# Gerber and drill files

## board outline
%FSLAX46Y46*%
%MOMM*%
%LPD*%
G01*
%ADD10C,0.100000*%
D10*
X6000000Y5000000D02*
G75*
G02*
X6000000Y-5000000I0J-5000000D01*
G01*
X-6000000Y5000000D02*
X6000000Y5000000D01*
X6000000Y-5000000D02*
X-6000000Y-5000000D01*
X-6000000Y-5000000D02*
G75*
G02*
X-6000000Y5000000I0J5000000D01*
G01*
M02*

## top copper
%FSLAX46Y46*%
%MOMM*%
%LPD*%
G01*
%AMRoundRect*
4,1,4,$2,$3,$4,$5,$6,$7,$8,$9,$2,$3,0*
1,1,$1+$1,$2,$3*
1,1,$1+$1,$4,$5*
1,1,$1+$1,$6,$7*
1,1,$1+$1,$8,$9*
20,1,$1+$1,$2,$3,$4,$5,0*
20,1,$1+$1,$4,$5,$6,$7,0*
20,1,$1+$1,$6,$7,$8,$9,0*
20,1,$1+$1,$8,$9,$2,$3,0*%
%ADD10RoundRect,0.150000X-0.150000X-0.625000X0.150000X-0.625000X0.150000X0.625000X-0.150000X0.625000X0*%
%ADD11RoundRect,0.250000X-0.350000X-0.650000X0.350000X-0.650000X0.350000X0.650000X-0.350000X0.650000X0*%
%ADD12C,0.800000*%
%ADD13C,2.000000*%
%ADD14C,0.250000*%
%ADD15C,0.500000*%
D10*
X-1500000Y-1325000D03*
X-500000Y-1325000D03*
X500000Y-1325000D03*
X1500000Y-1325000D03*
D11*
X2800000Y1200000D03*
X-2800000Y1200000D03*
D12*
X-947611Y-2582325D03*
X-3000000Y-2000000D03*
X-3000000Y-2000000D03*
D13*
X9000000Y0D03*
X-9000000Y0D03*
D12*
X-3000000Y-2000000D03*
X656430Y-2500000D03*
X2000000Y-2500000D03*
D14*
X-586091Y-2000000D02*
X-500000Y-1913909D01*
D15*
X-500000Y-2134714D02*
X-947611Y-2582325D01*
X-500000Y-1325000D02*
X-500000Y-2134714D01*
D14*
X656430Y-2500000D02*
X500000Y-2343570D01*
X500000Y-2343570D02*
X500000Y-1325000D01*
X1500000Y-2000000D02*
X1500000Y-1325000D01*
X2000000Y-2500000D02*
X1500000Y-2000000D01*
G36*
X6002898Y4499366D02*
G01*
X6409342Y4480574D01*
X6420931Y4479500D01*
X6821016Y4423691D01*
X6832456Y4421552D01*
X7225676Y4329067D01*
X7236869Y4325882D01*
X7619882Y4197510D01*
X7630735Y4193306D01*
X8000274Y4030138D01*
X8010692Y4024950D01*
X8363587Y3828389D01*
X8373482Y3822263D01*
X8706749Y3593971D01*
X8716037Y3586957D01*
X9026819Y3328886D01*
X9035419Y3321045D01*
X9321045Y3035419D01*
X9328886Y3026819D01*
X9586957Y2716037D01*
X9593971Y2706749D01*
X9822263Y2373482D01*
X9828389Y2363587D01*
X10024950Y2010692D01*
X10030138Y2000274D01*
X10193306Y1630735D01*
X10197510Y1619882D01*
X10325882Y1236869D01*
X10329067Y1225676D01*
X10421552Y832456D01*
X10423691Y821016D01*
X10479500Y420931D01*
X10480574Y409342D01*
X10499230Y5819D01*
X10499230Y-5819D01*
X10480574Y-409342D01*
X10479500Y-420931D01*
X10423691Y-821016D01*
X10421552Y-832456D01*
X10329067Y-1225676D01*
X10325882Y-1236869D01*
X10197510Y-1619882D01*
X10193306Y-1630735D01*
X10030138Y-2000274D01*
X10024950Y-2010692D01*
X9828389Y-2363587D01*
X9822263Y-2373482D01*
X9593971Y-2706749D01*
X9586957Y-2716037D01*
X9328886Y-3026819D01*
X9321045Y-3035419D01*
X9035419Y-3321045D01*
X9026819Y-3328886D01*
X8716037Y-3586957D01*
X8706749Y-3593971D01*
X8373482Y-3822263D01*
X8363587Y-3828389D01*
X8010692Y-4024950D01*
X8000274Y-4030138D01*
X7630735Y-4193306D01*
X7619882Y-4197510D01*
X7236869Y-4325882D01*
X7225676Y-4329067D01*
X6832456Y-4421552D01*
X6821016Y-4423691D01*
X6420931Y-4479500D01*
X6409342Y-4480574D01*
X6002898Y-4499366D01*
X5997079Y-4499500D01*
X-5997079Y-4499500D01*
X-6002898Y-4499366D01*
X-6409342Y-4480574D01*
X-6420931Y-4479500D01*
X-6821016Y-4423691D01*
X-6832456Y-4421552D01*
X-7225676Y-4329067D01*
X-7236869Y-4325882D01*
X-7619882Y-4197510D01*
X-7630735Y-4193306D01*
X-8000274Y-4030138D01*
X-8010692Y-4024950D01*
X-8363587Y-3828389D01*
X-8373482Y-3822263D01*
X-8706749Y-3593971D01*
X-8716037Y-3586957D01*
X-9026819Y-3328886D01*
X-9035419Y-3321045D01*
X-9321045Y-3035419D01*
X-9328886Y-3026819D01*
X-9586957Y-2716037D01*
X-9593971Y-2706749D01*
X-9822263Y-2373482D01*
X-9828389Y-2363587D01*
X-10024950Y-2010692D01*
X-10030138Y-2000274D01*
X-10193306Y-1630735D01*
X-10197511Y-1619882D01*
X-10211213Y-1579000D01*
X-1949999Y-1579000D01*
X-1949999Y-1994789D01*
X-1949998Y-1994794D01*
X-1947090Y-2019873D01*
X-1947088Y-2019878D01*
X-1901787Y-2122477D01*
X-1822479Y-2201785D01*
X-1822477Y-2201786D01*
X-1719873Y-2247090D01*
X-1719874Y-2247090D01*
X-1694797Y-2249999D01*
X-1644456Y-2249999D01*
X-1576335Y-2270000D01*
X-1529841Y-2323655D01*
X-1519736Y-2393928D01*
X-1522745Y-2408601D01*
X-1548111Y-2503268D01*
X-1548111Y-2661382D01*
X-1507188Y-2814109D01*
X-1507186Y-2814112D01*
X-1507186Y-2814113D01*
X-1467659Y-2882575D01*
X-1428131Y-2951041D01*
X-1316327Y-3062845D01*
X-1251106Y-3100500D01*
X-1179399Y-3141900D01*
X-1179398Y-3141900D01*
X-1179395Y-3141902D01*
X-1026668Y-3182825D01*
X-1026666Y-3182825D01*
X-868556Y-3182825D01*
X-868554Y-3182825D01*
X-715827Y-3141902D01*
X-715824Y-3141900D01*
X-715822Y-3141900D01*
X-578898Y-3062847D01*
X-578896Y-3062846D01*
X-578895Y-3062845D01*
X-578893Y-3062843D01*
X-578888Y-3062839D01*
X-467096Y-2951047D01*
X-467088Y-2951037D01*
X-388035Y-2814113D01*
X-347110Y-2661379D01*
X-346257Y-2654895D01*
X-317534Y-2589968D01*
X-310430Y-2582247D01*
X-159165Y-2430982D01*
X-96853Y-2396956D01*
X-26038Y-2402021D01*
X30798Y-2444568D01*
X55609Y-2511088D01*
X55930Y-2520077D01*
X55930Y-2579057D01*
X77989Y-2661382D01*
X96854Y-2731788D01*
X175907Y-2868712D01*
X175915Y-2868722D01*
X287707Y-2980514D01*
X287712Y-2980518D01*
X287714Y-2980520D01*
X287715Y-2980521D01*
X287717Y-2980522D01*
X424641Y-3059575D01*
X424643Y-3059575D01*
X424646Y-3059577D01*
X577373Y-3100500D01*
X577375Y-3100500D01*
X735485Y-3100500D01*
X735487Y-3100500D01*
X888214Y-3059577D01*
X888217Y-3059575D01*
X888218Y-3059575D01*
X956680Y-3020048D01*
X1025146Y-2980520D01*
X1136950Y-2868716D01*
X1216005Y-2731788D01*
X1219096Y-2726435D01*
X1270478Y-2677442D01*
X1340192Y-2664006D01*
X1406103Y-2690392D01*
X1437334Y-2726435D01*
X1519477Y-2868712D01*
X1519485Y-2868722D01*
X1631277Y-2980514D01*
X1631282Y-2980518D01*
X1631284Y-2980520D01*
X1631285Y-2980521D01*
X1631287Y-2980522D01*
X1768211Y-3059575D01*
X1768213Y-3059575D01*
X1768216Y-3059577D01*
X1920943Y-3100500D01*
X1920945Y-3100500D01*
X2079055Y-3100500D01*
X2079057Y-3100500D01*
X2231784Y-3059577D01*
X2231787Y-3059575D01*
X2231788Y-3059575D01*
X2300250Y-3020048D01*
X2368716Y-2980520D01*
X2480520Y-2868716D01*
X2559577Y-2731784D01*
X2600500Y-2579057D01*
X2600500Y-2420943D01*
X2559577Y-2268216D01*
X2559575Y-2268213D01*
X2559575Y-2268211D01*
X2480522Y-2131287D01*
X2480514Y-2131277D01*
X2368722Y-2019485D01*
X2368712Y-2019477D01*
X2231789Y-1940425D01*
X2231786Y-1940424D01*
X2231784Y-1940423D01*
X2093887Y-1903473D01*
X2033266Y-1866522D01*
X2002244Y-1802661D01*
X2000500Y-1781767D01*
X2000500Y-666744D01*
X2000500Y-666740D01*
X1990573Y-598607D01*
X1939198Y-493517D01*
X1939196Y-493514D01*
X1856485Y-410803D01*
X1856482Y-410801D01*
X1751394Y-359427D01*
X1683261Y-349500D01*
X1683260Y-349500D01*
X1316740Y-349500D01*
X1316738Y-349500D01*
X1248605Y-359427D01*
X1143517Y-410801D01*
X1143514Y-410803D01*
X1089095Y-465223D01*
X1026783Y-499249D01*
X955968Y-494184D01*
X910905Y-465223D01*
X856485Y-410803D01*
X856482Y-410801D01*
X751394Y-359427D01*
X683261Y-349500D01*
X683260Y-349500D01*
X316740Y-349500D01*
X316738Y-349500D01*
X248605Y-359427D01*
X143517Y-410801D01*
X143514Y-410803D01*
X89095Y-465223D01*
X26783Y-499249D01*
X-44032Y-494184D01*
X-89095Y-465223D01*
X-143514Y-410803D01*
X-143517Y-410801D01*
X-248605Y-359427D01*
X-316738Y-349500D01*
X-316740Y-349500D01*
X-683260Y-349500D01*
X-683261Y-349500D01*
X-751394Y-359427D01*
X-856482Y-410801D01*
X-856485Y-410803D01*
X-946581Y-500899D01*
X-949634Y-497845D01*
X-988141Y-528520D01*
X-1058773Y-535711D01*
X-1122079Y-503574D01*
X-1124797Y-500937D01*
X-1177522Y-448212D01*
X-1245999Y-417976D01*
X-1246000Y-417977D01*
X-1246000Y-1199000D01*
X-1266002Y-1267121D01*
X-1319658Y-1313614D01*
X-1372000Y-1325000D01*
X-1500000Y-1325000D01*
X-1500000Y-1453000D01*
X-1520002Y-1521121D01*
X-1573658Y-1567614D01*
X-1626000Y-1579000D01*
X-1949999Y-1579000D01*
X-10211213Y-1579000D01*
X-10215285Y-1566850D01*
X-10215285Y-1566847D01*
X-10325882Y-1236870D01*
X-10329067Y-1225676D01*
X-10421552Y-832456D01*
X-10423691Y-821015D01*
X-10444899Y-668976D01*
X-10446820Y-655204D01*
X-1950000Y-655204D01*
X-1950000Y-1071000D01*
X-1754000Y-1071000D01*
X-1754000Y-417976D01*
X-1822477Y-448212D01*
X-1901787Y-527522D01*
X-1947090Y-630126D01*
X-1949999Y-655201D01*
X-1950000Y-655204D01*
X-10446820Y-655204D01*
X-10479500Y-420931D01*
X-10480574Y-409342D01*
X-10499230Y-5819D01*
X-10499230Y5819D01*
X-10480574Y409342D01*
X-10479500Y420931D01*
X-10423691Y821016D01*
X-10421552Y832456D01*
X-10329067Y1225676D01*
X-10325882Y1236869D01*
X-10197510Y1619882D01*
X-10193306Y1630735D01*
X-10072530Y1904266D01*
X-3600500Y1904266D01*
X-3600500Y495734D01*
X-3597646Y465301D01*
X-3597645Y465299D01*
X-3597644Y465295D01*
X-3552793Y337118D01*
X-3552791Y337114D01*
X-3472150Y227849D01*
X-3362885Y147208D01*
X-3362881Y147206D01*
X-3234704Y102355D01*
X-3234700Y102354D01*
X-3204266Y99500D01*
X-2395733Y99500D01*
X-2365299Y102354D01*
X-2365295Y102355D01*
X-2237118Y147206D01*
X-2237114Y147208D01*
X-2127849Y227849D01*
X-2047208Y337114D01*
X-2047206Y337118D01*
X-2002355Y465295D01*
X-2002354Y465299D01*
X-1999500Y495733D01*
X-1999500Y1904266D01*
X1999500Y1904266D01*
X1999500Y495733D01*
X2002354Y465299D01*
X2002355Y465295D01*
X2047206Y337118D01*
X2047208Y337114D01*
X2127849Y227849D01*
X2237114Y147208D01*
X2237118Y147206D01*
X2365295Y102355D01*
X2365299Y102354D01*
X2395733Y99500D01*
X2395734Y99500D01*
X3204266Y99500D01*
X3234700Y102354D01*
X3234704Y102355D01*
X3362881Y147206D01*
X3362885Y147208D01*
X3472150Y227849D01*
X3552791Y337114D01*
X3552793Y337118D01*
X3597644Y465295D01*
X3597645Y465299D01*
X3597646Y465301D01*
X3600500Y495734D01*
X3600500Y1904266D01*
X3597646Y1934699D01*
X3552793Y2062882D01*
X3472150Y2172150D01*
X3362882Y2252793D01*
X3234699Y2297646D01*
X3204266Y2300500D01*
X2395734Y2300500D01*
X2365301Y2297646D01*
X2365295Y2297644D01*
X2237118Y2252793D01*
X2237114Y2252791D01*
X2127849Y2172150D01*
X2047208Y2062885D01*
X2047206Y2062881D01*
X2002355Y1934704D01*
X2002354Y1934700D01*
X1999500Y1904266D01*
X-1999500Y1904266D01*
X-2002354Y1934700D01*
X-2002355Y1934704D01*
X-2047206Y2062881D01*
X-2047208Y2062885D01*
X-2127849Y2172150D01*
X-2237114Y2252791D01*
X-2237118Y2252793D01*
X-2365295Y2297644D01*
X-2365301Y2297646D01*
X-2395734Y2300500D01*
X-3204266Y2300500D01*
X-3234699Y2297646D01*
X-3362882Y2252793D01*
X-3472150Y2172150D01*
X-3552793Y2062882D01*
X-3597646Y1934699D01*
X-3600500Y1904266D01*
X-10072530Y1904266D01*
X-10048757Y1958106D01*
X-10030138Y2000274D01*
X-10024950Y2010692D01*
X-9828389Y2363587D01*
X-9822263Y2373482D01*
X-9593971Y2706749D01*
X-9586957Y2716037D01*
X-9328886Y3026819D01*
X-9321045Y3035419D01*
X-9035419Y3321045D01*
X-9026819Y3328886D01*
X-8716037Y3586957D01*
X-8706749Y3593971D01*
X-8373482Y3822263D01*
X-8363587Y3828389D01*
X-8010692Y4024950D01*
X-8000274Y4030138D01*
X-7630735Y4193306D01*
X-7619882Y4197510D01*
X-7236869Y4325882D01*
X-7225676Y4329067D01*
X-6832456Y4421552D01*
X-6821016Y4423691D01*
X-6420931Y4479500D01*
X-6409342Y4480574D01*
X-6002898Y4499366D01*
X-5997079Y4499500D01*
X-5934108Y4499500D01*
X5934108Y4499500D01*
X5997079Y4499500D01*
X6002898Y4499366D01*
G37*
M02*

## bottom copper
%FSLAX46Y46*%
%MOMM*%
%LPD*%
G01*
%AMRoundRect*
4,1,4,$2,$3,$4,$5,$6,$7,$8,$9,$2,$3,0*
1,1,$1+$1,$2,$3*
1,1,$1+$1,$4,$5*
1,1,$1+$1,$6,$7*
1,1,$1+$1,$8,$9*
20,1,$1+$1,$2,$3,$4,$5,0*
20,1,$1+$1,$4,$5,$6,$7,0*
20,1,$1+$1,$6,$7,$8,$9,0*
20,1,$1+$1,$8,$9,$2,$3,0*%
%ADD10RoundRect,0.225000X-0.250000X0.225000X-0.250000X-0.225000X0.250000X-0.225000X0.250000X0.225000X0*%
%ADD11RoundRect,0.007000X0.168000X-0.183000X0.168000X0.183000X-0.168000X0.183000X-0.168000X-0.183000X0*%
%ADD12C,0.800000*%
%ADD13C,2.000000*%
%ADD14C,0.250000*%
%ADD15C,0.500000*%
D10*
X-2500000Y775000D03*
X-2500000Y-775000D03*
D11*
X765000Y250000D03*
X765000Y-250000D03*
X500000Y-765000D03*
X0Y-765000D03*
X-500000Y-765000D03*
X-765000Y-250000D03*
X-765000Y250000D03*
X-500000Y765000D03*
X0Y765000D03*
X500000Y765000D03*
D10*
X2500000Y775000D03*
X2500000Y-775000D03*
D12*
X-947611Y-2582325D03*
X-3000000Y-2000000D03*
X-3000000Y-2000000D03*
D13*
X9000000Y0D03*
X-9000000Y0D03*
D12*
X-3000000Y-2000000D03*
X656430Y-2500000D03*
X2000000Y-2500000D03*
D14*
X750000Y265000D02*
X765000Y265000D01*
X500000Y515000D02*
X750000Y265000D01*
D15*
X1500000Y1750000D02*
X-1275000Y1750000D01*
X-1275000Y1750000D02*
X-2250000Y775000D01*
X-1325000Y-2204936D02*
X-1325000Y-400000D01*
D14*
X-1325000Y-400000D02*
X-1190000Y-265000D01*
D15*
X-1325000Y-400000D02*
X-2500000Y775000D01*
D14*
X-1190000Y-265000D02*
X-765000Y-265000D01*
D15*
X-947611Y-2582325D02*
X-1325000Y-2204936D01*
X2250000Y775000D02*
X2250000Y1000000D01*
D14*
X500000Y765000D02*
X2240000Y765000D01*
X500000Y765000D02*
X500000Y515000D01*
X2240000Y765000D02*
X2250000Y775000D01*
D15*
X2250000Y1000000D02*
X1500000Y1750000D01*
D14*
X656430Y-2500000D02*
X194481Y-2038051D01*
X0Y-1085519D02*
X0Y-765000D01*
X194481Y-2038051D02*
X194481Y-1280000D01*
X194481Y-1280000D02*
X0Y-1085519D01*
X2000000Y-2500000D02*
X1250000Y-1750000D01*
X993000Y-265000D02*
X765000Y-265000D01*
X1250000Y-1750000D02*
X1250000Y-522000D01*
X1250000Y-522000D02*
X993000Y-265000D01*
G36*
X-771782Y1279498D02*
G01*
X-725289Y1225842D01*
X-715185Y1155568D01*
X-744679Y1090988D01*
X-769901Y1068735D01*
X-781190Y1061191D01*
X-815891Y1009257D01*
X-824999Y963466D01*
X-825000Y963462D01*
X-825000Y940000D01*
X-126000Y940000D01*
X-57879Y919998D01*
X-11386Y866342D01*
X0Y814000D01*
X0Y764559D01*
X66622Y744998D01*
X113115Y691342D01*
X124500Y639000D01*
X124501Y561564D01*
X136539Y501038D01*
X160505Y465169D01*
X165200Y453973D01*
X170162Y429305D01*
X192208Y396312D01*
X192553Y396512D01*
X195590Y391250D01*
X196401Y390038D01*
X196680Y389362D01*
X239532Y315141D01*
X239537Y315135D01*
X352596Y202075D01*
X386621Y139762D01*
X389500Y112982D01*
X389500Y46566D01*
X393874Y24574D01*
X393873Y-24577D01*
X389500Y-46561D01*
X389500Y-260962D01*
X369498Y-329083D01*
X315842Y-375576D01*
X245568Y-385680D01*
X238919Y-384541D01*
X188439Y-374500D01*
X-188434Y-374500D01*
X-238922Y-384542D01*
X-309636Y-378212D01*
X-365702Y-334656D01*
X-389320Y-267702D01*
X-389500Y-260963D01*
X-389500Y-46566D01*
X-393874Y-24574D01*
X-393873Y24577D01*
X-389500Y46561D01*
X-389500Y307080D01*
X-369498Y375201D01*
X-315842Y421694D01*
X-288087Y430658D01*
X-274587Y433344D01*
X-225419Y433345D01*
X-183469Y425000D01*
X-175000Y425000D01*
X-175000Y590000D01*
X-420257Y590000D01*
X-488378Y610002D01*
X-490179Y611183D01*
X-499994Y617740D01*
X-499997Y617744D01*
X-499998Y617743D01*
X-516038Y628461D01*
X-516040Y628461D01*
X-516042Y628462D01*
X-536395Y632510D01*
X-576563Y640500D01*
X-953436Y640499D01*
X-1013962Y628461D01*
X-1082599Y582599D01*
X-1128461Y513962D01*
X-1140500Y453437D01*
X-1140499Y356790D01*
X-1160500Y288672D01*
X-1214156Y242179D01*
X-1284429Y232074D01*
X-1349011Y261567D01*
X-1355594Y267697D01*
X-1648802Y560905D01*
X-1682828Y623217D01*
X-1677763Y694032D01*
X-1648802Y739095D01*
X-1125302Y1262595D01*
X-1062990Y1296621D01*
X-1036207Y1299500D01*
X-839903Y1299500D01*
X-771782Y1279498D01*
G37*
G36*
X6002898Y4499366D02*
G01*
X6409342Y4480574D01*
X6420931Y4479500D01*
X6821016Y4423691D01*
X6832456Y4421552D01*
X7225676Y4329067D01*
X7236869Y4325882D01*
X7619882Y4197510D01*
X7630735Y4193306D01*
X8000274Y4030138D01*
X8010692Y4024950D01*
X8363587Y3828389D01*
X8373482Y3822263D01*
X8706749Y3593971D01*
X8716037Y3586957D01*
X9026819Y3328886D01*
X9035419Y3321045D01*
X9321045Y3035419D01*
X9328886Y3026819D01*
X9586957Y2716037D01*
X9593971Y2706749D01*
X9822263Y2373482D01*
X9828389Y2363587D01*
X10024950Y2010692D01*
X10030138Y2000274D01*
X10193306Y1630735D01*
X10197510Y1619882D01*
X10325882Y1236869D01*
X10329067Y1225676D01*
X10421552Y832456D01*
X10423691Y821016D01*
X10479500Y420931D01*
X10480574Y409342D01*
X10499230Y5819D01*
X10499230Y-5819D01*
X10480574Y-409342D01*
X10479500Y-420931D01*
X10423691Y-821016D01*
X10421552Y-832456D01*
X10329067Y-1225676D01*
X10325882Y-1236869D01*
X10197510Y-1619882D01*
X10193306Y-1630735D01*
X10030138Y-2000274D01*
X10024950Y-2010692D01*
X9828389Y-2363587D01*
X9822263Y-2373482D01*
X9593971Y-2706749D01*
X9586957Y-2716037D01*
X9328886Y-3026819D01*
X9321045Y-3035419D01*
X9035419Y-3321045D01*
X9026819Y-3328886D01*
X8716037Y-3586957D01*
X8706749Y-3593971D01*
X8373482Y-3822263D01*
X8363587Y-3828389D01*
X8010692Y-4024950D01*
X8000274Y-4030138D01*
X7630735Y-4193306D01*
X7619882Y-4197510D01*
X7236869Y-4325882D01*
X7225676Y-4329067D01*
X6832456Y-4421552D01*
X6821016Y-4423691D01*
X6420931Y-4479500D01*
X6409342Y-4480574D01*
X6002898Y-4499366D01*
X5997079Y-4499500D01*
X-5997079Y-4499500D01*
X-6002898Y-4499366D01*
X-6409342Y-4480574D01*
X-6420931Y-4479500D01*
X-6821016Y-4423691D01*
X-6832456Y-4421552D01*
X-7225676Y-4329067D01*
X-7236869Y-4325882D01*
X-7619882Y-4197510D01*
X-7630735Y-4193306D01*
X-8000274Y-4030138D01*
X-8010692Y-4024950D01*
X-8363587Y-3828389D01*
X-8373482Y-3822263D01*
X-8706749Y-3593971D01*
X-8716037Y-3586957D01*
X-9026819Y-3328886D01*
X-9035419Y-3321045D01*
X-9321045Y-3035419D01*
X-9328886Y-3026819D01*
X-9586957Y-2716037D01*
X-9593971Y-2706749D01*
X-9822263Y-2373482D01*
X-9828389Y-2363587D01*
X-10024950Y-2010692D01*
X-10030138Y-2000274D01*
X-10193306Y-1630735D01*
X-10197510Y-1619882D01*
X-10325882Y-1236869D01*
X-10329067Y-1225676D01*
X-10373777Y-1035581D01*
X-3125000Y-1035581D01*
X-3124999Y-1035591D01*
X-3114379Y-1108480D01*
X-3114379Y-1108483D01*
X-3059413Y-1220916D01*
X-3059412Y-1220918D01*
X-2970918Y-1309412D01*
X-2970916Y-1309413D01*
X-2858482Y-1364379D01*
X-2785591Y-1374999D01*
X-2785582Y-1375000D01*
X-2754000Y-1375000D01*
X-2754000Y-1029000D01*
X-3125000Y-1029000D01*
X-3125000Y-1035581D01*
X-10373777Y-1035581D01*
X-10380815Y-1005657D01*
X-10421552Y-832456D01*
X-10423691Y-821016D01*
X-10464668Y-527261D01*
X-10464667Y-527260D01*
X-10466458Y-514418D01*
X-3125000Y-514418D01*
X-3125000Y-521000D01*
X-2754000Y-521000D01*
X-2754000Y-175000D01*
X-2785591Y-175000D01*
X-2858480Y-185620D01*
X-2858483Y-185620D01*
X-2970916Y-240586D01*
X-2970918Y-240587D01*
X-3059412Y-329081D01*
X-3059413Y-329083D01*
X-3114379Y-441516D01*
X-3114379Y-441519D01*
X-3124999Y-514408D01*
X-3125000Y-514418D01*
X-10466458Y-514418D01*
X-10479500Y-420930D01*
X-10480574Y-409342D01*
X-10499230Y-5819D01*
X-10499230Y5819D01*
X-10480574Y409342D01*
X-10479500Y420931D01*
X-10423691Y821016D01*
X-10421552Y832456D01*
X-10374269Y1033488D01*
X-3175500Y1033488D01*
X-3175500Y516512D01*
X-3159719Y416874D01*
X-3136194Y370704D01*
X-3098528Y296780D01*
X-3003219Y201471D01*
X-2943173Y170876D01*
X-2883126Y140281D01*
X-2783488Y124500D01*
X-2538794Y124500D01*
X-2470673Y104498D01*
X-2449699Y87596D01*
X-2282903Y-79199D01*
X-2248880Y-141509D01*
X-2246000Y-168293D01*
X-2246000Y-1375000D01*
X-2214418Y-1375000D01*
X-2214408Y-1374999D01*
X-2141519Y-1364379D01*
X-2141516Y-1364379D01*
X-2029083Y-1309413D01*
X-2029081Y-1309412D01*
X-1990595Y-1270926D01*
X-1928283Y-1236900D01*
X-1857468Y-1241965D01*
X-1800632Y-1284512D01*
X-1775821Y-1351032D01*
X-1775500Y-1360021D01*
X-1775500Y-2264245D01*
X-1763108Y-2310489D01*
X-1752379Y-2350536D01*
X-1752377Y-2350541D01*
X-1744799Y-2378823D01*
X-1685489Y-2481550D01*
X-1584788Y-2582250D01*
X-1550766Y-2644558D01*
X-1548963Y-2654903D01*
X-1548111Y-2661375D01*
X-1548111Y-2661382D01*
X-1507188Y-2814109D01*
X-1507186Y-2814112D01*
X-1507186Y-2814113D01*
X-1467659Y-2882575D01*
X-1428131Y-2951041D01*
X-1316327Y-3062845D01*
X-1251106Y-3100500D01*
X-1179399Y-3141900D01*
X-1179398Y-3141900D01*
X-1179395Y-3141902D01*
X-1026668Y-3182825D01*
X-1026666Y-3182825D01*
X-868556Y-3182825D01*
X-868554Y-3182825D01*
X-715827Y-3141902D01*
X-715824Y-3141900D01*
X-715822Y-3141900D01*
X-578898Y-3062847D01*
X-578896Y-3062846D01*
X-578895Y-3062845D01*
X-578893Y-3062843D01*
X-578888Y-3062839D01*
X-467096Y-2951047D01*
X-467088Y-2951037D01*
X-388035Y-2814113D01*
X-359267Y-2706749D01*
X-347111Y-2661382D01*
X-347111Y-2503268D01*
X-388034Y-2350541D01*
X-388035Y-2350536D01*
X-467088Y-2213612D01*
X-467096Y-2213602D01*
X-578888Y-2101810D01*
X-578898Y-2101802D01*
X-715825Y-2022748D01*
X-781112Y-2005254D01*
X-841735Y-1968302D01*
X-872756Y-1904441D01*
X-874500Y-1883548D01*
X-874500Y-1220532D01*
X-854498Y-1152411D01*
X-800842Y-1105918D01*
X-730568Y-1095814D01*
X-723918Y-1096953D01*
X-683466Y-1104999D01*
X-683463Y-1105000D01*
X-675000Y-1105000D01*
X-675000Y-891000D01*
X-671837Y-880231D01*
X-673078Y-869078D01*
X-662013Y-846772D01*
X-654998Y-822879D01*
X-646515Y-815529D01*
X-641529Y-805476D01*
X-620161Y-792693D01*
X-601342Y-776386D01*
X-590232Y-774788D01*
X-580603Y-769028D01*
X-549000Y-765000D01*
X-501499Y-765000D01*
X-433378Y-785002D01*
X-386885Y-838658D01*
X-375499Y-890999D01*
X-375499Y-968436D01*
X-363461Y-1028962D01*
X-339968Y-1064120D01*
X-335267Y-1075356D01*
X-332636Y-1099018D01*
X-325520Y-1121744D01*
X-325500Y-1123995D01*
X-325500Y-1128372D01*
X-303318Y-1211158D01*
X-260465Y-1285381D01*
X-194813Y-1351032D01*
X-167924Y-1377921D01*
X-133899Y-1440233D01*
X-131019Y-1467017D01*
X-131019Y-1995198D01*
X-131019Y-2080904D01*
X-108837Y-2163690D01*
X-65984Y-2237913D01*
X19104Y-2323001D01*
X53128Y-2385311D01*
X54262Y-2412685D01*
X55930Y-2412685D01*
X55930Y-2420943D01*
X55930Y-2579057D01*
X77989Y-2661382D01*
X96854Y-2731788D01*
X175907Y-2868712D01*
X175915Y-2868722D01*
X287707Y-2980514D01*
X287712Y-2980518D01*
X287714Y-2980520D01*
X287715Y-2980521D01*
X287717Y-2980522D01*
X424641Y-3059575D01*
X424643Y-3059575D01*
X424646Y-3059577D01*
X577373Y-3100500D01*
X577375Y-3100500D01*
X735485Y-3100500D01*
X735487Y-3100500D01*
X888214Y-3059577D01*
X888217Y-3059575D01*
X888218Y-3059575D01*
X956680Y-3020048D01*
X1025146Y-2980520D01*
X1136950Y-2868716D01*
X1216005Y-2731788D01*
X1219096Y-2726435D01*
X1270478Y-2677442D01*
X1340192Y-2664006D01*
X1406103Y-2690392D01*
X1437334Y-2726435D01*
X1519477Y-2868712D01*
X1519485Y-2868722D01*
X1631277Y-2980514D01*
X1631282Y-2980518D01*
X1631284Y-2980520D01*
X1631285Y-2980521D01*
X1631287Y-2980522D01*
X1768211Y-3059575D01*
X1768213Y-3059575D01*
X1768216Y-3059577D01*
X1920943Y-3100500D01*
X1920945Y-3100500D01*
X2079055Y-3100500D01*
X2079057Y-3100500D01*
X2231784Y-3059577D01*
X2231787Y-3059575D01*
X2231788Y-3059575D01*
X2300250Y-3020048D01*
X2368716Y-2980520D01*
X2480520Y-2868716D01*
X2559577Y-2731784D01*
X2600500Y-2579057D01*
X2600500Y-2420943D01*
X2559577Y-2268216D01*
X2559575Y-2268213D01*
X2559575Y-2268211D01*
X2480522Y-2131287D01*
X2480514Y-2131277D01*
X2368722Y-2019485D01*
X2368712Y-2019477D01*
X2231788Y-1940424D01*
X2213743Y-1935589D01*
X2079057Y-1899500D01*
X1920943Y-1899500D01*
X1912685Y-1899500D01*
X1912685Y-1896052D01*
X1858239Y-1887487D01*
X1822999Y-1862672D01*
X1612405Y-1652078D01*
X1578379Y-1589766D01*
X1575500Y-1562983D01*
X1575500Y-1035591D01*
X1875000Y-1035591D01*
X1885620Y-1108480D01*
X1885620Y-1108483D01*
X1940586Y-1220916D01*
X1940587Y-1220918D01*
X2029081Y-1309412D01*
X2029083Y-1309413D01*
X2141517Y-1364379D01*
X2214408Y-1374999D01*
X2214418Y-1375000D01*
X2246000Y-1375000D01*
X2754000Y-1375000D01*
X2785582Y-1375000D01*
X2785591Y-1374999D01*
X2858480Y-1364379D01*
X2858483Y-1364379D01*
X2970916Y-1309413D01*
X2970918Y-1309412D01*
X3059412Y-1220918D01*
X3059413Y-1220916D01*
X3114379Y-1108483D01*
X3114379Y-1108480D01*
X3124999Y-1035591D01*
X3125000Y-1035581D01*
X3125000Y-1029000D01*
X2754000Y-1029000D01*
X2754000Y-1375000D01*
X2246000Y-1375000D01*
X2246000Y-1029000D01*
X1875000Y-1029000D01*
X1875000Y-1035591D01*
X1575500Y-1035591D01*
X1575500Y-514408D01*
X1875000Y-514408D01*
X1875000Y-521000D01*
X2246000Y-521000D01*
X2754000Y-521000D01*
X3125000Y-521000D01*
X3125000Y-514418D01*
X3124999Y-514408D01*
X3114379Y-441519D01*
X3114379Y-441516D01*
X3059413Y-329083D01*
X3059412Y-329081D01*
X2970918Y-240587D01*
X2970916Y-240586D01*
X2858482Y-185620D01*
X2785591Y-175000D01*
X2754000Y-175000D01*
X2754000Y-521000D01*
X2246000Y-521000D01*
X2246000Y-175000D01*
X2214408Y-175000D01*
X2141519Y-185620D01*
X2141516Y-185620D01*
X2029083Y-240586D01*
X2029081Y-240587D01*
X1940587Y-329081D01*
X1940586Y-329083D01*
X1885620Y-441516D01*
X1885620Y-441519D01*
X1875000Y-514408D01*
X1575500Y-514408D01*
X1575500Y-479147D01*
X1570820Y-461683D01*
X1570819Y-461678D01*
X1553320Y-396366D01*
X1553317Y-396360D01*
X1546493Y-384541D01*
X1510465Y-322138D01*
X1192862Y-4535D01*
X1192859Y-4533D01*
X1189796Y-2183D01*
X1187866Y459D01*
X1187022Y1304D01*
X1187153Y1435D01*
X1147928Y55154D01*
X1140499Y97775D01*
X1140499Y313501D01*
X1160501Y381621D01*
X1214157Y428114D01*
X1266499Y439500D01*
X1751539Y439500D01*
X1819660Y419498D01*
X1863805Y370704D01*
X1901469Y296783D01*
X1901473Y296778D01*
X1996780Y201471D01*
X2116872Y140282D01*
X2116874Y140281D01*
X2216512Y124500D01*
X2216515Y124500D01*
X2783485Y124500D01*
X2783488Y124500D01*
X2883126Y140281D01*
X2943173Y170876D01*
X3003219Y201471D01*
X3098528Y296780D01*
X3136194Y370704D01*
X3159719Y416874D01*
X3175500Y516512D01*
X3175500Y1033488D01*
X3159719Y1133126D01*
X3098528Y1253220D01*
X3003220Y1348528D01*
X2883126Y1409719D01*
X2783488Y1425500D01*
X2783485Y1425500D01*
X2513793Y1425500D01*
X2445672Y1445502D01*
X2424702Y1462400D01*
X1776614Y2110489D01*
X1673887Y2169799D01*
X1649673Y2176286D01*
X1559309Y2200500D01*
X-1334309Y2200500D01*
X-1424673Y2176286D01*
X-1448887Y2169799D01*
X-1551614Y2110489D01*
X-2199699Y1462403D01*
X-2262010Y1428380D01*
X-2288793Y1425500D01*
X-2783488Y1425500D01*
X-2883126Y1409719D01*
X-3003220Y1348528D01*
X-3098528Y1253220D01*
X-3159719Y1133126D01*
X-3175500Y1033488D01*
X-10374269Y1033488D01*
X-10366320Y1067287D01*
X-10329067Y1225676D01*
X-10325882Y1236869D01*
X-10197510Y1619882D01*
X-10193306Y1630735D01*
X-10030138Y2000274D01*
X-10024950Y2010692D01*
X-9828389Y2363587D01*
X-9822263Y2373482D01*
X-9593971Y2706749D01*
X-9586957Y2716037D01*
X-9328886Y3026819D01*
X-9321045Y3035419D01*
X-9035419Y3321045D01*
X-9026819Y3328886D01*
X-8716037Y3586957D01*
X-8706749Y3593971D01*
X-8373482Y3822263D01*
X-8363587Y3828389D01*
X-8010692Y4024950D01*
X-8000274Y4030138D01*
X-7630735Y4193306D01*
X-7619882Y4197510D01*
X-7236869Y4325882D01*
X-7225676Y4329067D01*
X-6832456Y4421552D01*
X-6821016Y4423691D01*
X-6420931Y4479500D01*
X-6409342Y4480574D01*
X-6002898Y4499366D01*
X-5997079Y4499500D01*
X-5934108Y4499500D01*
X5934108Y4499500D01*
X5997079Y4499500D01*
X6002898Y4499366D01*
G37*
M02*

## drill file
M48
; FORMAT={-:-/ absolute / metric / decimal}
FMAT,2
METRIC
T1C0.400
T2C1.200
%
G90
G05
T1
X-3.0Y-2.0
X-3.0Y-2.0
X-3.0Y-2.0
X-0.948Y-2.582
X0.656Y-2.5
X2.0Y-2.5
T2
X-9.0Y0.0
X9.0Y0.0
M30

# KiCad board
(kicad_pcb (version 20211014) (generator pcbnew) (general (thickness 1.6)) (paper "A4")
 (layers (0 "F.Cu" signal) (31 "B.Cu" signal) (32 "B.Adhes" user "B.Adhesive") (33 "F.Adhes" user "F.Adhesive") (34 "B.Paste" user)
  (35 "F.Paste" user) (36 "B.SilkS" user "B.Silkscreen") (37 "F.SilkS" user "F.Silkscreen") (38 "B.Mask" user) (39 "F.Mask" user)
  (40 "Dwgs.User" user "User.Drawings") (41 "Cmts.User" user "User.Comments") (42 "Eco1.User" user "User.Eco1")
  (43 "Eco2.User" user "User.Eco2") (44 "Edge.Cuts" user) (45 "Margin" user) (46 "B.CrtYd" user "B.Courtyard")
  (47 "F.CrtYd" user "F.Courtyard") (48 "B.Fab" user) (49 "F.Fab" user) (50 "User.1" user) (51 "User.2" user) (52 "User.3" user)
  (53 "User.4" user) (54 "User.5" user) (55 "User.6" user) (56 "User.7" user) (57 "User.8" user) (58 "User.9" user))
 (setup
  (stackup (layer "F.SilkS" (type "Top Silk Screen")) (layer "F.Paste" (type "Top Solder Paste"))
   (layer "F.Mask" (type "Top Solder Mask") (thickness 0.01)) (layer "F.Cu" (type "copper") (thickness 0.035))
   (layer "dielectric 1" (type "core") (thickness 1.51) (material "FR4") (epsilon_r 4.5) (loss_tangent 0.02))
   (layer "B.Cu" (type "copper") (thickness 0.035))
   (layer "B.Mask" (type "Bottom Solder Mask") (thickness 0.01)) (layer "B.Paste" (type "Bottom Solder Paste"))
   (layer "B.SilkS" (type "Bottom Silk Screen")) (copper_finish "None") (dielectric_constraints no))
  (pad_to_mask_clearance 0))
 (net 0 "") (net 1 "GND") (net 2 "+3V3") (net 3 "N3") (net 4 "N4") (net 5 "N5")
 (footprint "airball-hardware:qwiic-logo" (layer "F.Cu") (at 5 0 90)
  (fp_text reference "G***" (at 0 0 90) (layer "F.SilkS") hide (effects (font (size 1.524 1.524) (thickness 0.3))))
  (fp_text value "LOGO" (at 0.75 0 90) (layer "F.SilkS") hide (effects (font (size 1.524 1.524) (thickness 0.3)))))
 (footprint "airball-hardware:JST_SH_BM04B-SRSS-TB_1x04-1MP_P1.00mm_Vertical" (layer "F.Cu") (at 0 0)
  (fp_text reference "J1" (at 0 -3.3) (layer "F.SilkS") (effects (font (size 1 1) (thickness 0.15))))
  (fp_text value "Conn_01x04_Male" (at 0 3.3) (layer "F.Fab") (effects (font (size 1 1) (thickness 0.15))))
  (pad "1" smd roundrect (at -1.5 1.325) (size 0.6 1.55) (layers "F.Cu" "F.Paste" "F.Mask") (roundrect_rratio 0.25) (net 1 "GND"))
  (pad "2" smd roundrect (at -0.5 1.325) (size 0.6 1.55) (layers "F.Cu" "F.Paste" "F.Mask") (roundrect_rratio 0.25) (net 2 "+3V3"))
  (pad "3" smd roundrect (at 0.5 1.325) (size 0.6 1.55) (layers "F.Cu" "F.Paste" "F.Mask") (roundrect_rratio 0.25) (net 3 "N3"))
  (pad "4" smd roundrect (at 1.5 1.325) (size 0.6 1.55) (layers "F.Cu" "F.Paste" "F.Mask") (roundrect_rratio 0.25) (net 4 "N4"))
  (pad "MP" smd roundrect (at 2.8 -1.2) (size 1.2 1.8) (layers "F.Cu" "F.Paste" "F.Mask") (roundrect_rratio 0.208333))
  (pad "MP" smd roundrect (at -2.8 -1.2) (size 1.2 1.8) (layers "F.Cu" "F.Paste" "F.Mask") (roundrect_rratio 0.208333)))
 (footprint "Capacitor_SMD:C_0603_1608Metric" (layer "B.Cu") (at -2.5 0 -90)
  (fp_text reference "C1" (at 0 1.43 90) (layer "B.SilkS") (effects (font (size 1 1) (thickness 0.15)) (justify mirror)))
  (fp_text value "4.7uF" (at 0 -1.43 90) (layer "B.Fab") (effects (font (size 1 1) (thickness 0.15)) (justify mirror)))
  (pad "1" smd roundrect (at -0.775 0 270) (size 0.9 0.95) (layers "B.Cu" "B.Paste" "B.Mask") (roundrect_rratio 0.25) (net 2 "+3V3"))
  (pad "2" smd roundrect (at 0.775 0 270) (size 0.9 0.95) (layers "B.Cu" "B.Paste" "B.Mask") (roundrect_rratio 0.25) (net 1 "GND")))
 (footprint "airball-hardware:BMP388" (layer "B.Cu") (at 0 0 180)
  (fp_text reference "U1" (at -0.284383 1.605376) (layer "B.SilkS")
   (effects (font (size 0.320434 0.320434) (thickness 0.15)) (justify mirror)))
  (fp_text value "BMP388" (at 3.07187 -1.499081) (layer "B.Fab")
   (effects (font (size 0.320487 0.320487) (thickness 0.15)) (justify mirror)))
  (pad "1" smd roundrect (at -0.765 0.25 90) (size 0.38 0.35) (layers "B.Cu" "B.Paste" "B.Mask") (roundrect_rratio 0.02) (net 2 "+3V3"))
  (pad "2" smd roundrect (at -0.765 -0.25 90) (size 0.38 0.35) (layers "B.Cu" "B.Paste" "B.Mask") (roundrect_rratio 0.02) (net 4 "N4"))
  (pad "3" smd roundrect (at -0.5 -0.765 90) (size 0.38 0.35) (layers "B.Cu" "B.Paste" "B.Mask") (roundrect_rratio 0.02) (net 1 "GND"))
  (pad "4" smd roundrect (at 0 -0.765 90) (size 0.38 0.35) (layers "B.Cu" "B.Paste" "B.Mask") (roundrect_rratio 0.02) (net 3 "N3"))
  (pad "5" smd roundrect (at 0.5 -0.765 90) (size 0.38 0.35) (layers "B.Cu" "B.Paste" "B.Mask") (roundrect_rratio 0.02) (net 1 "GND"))
  (pad "6" smd roundrect (at 0.765 -0.25 90) (size 0.38 0.35) (layers "B.Cu" "B.Paste" "B.Mask") (roundrect_rratio 0.02) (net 2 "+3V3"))
  (pad "7" smd roundrect (at 0.765 0.25 90) (size 0.38 0.35) (layers "B.Cu" "B.Paste" "B.Mask") (roundrect_rratio 0.02) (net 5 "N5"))
  (pad "8" smd roundrect (at 0.5 0.765 90) (size 0.38 0.35) (layers "B.Cu" "B.Paste" "B.Mask") (roundrect_rratio 0.02) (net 1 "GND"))
  (pad "9" smd roundrect (at 0 0.765 90) (size 0.38 0.35) (layers "B.Cu" "B.Paste" "B.Mask") (roundrect_rratio 0.02) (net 1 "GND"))
  (pad "10" smd roundrect (at -0.5 0.765 90) (size 0.38 0.35) (layers "B.Cu" "B.Paste" "B.Mask") (roundrect_rratio 0.02) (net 2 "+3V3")))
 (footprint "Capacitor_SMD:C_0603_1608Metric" (layer "B.Cu") (at 2.5 0 -90)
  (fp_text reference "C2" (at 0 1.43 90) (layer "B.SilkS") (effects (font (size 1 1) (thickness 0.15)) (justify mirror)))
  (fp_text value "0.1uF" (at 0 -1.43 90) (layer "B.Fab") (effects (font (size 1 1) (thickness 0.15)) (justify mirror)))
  (pad "1" smd roundrect (at -0.775 0 270) (size 0.9 0.95) (layers "B.Cu" "B.Paste" "B.Mask") (roundrect_rratio 0.25) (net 2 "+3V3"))
  (pad "2" smd roundrect (at 0.775 0 270) (size 0.9 0.95) (layers "B.Cu" "B.Paste" "B.Mask") (roundrect_rratio 0.25) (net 1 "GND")))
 (gr_arc (start 6 -5) (mid 11 0) (end 6 5) (layer "Edge.Cuts") (width 0.1))
 (gr_line (start -6 -5) (end 6 -5) (layer "Edge.Cuts") (width 0.1))
 (gr_line (start 6 5) (end -6 5) (layer "Edge.Cuts") (width 0.1))
 (gr_arc (start -6 5) (mid -11 0) (end -6 -5) (layer "Edge.Cuts") (width 0.1))
 (segment (start -0.586091 2) (end -0.5 1.913909) (width 0.25) (layer "F.Cu") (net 2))
 (segment (start -0.5 2.134714) (end -0.947611 2.582325) (width 0.5) (layer "F.Cu") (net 2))
 (segment (start -0.5 1.325) (end -0.5 2.134714) (width 0.5) (layer "F.Cu") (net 2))
 (via (at -0.947611 2.582325) (size 0.8) (drill 0.4) (layers "F.Cu" "B.Cu") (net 2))
 (segment (start 0.75 -0.265) (end 0.765 -0.265) (width 0.25) (layer "B.Cu") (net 2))
 (segment (start 0.5 -0.515) (end 0.75 -0.265) (width 0.25) (layer "B.Cu") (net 2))
 (segment (start 1.5 -1.75) (end -1.275 -1.75) (width 0.5) (layer "B.Cu") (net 2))
 (segment (start -1.275 -1.75) (end -2.25 -0.775) (width 0.5) (layer "B.Cu") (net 2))
 (segment (start -1.325 2.204936) (end -1.325 0.4) (width 0.5) (layer "B.Cu") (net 2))
 (segment (start -1.325 0.4) (end -1.19 0.265) (width 0.25) (layer "B.Cu") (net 2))
 (segment (start -1.325 0.4) (end -2.5 -0.775) (width 0.5) (layer "B.Cu") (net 2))
 (segment (start -1.19 0.265) (end -0.765 0.265) (width 0.25) (layer "B.Cu") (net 2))
 (segment (start -0.947611 2.582325) (end -1.325 2.204936) (width 0.5) (layer "B.Cu") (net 2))
 (segment (start 2.25 -0.775) (end 2.25 -1) (width 0.5) (layer "B.Cu") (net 2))
 (segment (start 0.5 -0.765) (end 2.24 -0.765) (width 0.25) (layer "B.Cu") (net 2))
 (segment (start 0.5 -0.765) (end 0.5 -0.515) (width 0.25) (layer "B.Cu") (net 2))
 (segment (start 2.24 -0.765) (end 2.25 -0.775) (width 0.25) (layer "B.Cu") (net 2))
 (segment (start 2.25 -1) (end 1.5 -1.75) (width 0.5) (layer "B.Cu") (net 2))
 (via (at -3 2) (size 0.8) (drill 0.4) (layers "F.Cu" "B.Cu") (free) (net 1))
 (via (at -3 2) (size 0.8) (drill 0.4) (layers "F.Cu" "B.Cu") (free) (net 1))
 (via (at 9 0) (size 2) (drill 1.2) (layers "F.Cu" "B.Cu") (free) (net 1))
 (via (at -9 0) (size 2) (drill 1.2) (layers "F.Cu" "B.Cu") (free) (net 1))
 (via (at -3 2) (size 0.8) (drill 0.4) (layers "F.Cu" "B.Cu") (free) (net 1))
 (segment (start 0.65643 2.5) (end 0.5 2.34357) (width 0.25) (layer "F.Cu") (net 3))
 (segment (start 0.5 2.34357) (end 0.5 1.325) (width 0.25) (layer "F.Cu") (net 3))
 (via (at 0.65643 2.5) (size 0.8) (drill 0.4) (layers "F.Cu" "B.Cu") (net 3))
 (segment (start 0.65643 2.5) (end 0.194481 2.038051) (width 0.25) (layer "B.Cu") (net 3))
 (segment (start 0 1.085519) (end 0 0.765) (width 0.25) (layer "B.Cu") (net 3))
 (segment (start 0.194481 2.038051) (end 0.194481 1.28) (width 0.25) (layer "B.Cu") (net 3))
 (segment (start 0.194481 1.28) (end 0 1.085519) (width 0.25) (layer "B.Cu") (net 3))
 (segment (start 1.5 2) (end 1.5 1.325) (width 0.25) (layer "F.Cu") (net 4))
 (segment (start 2 2.5) (end 1.5 2) (width 0.25) (layer "F.Cu") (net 4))
 (via (at 2 2.5) (size 0.8) (drill 0.4) (layers "F.Cu" "B.Cu") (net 4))
 (segment (start 2 2.5) (end 1.25 1.75) (width 0.25) (layer "B.Cu") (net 4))
 (segment (start 0.993 0.265) (end 0.765 0.265) (width 0.25) (layer "B.Cu") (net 4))
 (segment (start 1.25 1.75) (end 1.25 0.522) (width 0.25) (layer "B.Cu") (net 4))
 (segment (start 1.25 0.522) (end 0.993 0.265) (width 0.25) (layer "B.Cu") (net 4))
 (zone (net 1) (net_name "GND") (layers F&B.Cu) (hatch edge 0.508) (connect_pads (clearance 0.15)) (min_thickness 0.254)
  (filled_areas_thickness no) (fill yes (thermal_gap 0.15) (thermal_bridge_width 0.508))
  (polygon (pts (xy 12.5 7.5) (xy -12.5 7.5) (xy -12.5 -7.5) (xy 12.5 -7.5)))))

